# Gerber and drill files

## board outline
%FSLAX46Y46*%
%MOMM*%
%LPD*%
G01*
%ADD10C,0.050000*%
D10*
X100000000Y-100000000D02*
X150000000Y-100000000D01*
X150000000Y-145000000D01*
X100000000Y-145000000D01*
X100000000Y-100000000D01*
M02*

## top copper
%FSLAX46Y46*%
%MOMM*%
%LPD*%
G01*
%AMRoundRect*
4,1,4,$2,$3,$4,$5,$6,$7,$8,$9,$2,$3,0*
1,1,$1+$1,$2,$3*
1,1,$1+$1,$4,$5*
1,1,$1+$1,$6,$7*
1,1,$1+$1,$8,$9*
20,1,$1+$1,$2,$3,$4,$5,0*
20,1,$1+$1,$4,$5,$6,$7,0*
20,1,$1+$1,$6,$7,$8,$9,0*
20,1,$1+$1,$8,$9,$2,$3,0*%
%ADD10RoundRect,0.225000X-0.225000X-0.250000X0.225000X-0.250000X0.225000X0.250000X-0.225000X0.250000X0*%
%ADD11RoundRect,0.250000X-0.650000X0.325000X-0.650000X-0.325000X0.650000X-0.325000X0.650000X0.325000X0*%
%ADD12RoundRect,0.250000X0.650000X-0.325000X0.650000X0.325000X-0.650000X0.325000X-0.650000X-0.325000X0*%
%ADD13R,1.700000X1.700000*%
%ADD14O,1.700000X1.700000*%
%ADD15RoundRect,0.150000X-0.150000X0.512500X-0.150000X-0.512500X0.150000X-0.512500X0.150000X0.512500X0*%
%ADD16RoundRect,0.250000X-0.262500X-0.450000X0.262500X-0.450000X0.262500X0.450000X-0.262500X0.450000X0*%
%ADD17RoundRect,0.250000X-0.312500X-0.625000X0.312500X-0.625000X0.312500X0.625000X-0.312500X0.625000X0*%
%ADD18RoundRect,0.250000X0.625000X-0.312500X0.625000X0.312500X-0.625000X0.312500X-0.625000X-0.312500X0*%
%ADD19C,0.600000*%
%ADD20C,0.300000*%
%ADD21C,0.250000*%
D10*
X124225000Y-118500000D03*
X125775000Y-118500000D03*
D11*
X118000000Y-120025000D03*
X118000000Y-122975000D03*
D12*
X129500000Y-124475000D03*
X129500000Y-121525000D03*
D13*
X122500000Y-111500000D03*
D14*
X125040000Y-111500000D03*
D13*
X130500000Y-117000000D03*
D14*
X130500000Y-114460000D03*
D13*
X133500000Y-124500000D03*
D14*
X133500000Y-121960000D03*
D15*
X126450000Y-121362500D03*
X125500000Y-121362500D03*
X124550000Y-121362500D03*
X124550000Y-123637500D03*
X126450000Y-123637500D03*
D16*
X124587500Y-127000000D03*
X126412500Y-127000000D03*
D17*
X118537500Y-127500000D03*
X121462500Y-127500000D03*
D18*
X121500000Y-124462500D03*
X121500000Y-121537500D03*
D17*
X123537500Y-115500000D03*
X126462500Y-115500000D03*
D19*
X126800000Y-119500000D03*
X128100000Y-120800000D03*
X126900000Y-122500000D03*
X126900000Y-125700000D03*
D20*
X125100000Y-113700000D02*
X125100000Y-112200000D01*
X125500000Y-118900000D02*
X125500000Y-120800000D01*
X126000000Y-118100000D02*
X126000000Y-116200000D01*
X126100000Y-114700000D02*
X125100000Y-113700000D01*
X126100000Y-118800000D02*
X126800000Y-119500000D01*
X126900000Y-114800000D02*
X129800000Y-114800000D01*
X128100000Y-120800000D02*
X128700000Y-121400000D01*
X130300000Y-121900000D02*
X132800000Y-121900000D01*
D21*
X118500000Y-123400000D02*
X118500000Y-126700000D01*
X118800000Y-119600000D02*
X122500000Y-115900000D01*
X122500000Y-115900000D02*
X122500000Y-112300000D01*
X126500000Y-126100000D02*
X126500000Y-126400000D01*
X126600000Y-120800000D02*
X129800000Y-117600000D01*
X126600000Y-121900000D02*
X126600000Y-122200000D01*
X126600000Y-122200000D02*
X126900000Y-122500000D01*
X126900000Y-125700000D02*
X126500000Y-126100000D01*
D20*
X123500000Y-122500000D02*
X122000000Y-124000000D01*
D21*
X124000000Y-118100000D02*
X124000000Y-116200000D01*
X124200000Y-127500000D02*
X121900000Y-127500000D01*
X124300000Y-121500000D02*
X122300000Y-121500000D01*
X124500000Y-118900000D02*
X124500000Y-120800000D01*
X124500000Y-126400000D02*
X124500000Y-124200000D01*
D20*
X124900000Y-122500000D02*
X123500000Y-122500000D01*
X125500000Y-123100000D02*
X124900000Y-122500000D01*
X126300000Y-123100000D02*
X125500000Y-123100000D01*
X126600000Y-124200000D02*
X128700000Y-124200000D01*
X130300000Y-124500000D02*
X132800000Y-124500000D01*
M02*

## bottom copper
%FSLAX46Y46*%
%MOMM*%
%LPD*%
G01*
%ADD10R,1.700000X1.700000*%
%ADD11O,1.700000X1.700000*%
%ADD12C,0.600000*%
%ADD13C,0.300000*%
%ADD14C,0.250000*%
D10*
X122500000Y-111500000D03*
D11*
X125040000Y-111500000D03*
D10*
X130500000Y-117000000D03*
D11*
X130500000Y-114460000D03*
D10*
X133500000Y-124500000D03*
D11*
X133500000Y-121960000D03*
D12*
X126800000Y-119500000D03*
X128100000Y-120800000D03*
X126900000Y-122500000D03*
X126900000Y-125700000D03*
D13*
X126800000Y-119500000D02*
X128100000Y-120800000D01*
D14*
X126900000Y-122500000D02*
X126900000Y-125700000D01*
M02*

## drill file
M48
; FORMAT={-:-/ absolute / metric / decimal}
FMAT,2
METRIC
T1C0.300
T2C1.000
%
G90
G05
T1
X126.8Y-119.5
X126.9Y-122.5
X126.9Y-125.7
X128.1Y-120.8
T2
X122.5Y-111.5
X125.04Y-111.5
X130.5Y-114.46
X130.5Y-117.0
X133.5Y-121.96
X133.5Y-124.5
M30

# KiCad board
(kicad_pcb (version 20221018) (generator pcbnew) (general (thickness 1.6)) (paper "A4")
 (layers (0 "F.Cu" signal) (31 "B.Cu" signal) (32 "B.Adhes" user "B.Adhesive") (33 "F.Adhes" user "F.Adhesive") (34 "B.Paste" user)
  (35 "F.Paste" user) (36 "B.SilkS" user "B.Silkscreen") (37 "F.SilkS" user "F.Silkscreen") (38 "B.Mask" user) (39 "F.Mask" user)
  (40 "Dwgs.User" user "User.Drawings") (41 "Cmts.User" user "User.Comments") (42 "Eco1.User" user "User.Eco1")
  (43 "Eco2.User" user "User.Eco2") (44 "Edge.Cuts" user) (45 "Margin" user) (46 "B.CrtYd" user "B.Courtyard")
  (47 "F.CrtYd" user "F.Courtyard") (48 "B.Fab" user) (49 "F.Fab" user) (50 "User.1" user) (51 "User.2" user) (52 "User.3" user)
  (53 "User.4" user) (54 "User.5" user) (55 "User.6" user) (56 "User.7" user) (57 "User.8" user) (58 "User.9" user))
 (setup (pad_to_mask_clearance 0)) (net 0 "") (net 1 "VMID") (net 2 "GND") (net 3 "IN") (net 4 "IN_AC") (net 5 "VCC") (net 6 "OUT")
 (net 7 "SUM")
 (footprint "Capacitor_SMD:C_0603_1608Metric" (layer "F.Cu") (at 125 118.5)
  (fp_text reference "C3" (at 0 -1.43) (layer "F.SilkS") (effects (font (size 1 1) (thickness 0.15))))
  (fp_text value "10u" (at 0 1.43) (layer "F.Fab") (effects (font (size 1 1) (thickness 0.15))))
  (pad "1" smd roundrect (at -0.775 0) (size 0.9 0.95) (layers "F.Cu" "F.Paste" "F.Mask") (roundrect_rratio 0.25) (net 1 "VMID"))
  (pad "2" smd roundrect (at 0.775 0) (size 0.9 0.95) (layers "F.Cu" "F.Paste" "F.Mask") (roundrect_rratio 0.25) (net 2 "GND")))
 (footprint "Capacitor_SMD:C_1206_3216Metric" (layer "F.Cu") (at 118 121.5 -90)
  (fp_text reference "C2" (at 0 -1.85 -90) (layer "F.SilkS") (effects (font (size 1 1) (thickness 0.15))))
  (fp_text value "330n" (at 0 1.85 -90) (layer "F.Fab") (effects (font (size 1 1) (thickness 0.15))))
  (pad "1" smd roundrect (at -1.475 0 270) (size 1.15 1.8) (layers "F.Cu" "F.Paste" "F.Mask") (roundrect_rratio 0.217391) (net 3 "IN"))
  (pad "2" smd roundrect (at 1.475 0 270) (size 1.15 1.8) (layers "F.Cu" "F.Paste" "F.Mask") (roundrect_rratio 0.217391) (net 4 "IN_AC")))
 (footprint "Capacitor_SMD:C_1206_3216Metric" (layer "F.Cu") (at 129.5 123 90)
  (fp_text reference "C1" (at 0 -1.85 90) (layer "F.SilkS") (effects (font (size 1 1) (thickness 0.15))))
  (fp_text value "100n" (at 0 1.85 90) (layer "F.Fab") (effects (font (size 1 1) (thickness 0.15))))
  (pad "1" smd roundrect (at -1.475 0 90) (size 1.15 1.8) (layers "F.Cu" "F.Paste" "F.Mask") (roundrect_rratio 0.217391) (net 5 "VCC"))
  (pad "2" smd roundrect (at 1.475 0 90) (size 1.15 1.8) (layers "F.Cu" "F.Paste" "F.Mask") (roundrect_rratio 0.217391) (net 2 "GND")))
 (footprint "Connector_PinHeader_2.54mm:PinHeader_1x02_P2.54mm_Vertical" (layer "F.Cu") (at 122.5 111.5 90)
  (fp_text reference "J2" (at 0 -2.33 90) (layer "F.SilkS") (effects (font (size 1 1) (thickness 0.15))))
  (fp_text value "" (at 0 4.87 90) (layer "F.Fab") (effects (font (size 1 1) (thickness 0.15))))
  (pad "1" thru_hole rect (at 0 0 90) (size 1.7 1.7) (drill 1) (layers "*.Cu" "*.Mask") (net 3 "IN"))
  (pad "2" thru_hole oval (at 0 2.54 90) (size 1.7 1.7) (drill 1) (layers "*.Cu" "*.Mask") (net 2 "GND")))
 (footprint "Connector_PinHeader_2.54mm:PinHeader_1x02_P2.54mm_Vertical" (layer "F.Cu") (at 130.5 117 180)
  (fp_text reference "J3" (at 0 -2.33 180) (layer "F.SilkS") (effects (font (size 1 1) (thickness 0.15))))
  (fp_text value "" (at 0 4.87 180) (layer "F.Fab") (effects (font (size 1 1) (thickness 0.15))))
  (pad "1" thru_hole rect (at 0 0 180) (size 1.7 1.7) (drill 1) (layers "*.Cu" "*.Mask") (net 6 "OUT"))
  (pad "2" thru_hole oval (at 0 2.54 180) (size 1.7 1.7) (drill 1) (layers "*.Cu" "*.Mask") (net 2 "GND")))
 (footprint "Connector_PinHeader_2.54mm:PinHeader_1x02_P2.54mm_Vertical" (layer "F.Cu") (at 133.5 124.5 180)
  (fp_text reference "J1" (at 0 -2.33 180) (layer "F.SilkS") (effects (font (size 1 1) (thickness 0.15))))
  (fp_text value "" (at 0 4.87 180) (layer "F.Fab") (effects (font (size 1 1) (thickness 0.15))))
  (pad "1" thru_hole rect (at 0 0 180) (size 1.7 1.7) (drill 1) (layers "*.Cu" "*.Mask") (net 5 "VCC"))
  (pad "2" thru_hole oval (at 0 2.54 180) (size 1.7 1.7) (drill 1) (layers "*.Cu" "*.Mask") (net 2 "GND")))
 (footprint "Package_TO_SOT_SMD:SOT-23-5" (layer "F.Cu") (at 125.5 122.5 -90)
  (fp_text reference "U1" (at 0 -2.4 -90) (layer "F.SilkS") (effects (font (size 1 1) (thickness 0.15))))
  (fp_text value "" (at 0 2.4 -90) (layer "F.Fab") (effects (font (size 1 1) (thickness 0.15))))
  (pad "1" smd roundrect (at -1.1375 -0.95 270) (size 1.325 0.6) (layers "F.Cu" "F.Paste" "F.Mask") (roundrect_rratio 0.25) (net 6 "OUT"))
  (pad "2" smd roundrect (at -1.1375 0 270) (size 1.325 0.6) (layers "F.Cu" "F.Paste" "F.Mask") (roundrect_rratio 0.25) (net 2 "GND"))
  (pad "3" smd roundrect (at -1.1375 0.95 270) (size 1.325 0.6) (layers "F.Cu" "F.Paste" "F.Mask") (roundrect_rratio 0.25) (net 1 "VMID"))
  (pad "4" smd roundrect (at 1.1375 0.95 270) (size 1.325 0.6) (layers "F.Cu" "F.Paste" "F.Mask") (roundrect_rratio 0.25) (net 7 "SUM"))
  (pad "5" smd roundrect (at 1.1375 -0.95 270) (size 1.325 0.6) (layers "F.Cu" "F.Paste" "F.Mask") (roundrect_rratio 0.25) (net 5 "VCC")))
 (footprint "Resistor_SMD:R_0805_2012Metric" (layer "F.Cu") (at 125.5 127)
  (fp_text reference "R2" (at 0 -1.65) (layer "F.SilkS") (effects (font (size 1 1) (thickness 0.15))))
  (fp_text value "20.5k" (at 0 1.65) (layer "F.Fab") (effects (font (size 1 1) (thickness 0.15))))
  (pad "1" smd roundrect (at -0.9125 0) (size 1.025 1.4) (layers "F.Cu" "F.Paste" "F.Mask") (roundrect_rratio 0.243902) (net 7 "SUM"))
  (pad "2" smd roundrect (at 0.9125 0) (size 1.025 1.4) (layers "F.Cu" "F.Paste" "F.Mask") (roundrect_rratio 0.243902) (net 6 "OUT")))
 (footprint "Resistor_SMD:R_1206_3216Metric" (layer "F.Cu") (at 120 127.5)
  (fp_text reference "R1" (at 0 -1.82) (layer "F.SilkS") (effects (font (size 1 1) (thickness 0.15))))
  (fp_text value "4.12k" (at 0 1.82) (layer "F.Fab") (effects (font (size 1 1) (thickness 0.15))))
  (pad "1" smd roundrect (at -1.4625 0) (size 1.125 1.75) (layers "F.Cu" "F.Paste" "F.Mask") (roundrect_rratio 0.222222) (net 4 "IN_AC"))
  (pad "2" smd roundrect (at 1.4625 0) (size 1.125 1.75) (layers "F.Cu" "F.Paste" "F.Mask") (roundrect_rratio 0.222222) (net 7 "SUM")))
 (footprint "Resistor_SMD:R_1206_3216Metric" (layer "F.Cu") (at 121.5 123 90)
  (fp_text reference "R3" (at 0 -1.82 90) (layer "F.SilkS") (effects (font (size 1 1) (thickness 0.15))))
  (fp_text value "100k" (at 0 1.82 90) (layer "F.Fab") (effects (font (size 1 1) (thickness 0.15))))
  (pad "1" smd roundrect (at -1.4625 0 90) (size 1.125 1.75) (layers "F.Cu" "F.Paste" "F.Mask") (roundrect_rratio 0.222222) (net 5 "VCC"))
  (pad "2" smd roundrect (at 1.4625 0 90) (size 1.125 1.75) (layers "F.Cu" "F.Paste" "F.Mask") (roundrect_rratio 0.222222) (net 1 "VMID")))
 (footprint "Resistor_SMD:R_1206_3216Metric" (layer "F.Cu") (at 125 115.5)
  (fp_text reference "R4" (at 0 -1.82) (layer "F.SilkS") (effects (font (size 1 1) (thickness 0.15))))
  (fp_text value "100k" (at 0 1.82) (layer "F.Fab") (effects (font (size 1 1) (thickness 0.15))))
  (pad "1" smd roundrect (at -1.4625 0) (size 1.125 1.75) (layers "F.Cu" "F.Paste" "F.Mask") (roundrect_rratio 0.222222) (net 1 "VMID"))
  (pad "2" smd roundrect (at 1.4625 0) (size 1.125 1.75) (layers "F.Cu" "F.Paste" "F.Mask") (roundrect_rratio 0.222222) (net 2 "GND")))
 (gr_rect (start 100 100) (end 150 145) (stroke (width 0.05) (type default)) (fill none) (layer "Edge.Cuts"))
 (segment (start 125.1 113.7) (end 125.1 112.2) (width 0.3) (layer "F.Cu") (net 2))
 (segment (start 125.5 118.9) (end 125.5 120.8) (width 0.3) (layer "F.Cu") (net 2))
 (segment (start 126 118.1) (end 126 116.2) (width 0.3) (layer "F.Cu") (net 2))
 (segment (start 126.1 114.7) (end 125.1 113.7) (width 0.3) (layer "F.Cu") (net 2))
 (segment (start 126.1 118.8) (end 126.8 119.5) (width 0.3) (layer "F.Cu") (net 2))
 (segment (start 126.9 114.8) (end 129.8 114.8) (width 0.3) (layer "F.Cu") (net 2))
 (segment (start 128.1 120.8) (end 128.7 121.4) (width 0.3) (layer "F.Cu") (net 2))
 (segment (start 130.3 121.9) (end 132.8 121.9) (width 0.3) (layer "F.Cu") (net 2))
 (via (at 126.8 119.5) (size 0.6) (drill 0.3) (layers "F.Cu" "B.Cu") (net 2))
 (via (at 128.1 120.8) (size 0.6) (drill 0.3) (layers "F.Cu" "B.Cu") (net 2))
 (segment (start 118.5 123.4) (end 118.5 126.7) (width 0.25) (layer "F.Cu") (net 4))
 (segment (start 118.8 119.6) (end 122.5 115.9) (width 0.25) (layer "F.Cu") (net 3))
 (segment (start 122.5 115.9) (end 122.5 112.3) (width 0.25) (layer "F.Cu") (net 3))
 (segment (start 126.5 126.1) (end 126.5 126.4) (width 0.25) (layer "F.Cu") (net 6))
 (segment (start 126.6 120.8) (end 129.8 117.6) (width 0.25) (layer "F.Cu") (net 6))
 (segment (start 126.6 121.9) (end 126.6 122.2) (width 0.25) (layer "F.Cu") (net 6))
 (segment (start 126.6 122.2) (end 126.9 122.5) (width 0.25) (layer "F.Cu") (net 6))
 (segment (start 126.8 119.5) (end 128.1 120.8) (width 0.3) (layer "B.Cu") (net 2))
 (segment (start 126.9 125.7) (end 126.5 126.1) (width 0.25) (layer "F.Cu") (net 6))
 (via (at 126.9 122.5) (size 0.6) (drill 0.3) (layers "F.Cu" "B.Cu") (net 6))
 (via (at 126.9 125.7) (size 0.6) (drill 0.3) (layers "F.Cu" "B.Cu") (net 6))
 (segment (start 123.5 122.5) (end 122 124) (width 0.3) (layer "F.Cu") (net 5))
 (segment (start 124 118.1) (end 124 116.2) (width 0.25) (layer "F.Cu") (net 1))
 (segment (start 124.2 127.5) (end 121.9 127.5) (width 0.25) (layer "F.Cu") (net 7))
 (segment (start 124.3 121.5) (end 122.3 121.5) (width 0.25) (layer "F.Cu") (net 1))
 (segment (start 124.5 118.9) (end 124.5 120.8) (width 0.25) (layer "F.Cu") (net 1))
 (segment (start 124.5 126.4) (end 124.5 124.2) (width 0.25) (layer "F.Cu") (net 7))
 (segment (start 124.9 122.5) (end 123.5 122.5) (width 0.3) (layer "F.Cu") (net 5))
 (segment (start 125.5 123.1) (end 124.9 122.5) (width 0.3) (layer "F.Cu") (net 5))
 (segment (start 126.3 123.1) (end 125.5 123.1) (width 0.3) (layer "F.Cu") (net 5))
 (segment (start 126.6 124.2) (end 128.7 124.2) (width 0.3) (layer "F.Cu") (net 5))
 (segment (start 126.9 122.5) (end 126.9 125.7) (width 0.25) (layer "B.Cu") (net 6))
 (segment (start 130.3 124.5) (end 132.8 124.5) (width 0.3) (layer "F.Cu") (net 5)))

